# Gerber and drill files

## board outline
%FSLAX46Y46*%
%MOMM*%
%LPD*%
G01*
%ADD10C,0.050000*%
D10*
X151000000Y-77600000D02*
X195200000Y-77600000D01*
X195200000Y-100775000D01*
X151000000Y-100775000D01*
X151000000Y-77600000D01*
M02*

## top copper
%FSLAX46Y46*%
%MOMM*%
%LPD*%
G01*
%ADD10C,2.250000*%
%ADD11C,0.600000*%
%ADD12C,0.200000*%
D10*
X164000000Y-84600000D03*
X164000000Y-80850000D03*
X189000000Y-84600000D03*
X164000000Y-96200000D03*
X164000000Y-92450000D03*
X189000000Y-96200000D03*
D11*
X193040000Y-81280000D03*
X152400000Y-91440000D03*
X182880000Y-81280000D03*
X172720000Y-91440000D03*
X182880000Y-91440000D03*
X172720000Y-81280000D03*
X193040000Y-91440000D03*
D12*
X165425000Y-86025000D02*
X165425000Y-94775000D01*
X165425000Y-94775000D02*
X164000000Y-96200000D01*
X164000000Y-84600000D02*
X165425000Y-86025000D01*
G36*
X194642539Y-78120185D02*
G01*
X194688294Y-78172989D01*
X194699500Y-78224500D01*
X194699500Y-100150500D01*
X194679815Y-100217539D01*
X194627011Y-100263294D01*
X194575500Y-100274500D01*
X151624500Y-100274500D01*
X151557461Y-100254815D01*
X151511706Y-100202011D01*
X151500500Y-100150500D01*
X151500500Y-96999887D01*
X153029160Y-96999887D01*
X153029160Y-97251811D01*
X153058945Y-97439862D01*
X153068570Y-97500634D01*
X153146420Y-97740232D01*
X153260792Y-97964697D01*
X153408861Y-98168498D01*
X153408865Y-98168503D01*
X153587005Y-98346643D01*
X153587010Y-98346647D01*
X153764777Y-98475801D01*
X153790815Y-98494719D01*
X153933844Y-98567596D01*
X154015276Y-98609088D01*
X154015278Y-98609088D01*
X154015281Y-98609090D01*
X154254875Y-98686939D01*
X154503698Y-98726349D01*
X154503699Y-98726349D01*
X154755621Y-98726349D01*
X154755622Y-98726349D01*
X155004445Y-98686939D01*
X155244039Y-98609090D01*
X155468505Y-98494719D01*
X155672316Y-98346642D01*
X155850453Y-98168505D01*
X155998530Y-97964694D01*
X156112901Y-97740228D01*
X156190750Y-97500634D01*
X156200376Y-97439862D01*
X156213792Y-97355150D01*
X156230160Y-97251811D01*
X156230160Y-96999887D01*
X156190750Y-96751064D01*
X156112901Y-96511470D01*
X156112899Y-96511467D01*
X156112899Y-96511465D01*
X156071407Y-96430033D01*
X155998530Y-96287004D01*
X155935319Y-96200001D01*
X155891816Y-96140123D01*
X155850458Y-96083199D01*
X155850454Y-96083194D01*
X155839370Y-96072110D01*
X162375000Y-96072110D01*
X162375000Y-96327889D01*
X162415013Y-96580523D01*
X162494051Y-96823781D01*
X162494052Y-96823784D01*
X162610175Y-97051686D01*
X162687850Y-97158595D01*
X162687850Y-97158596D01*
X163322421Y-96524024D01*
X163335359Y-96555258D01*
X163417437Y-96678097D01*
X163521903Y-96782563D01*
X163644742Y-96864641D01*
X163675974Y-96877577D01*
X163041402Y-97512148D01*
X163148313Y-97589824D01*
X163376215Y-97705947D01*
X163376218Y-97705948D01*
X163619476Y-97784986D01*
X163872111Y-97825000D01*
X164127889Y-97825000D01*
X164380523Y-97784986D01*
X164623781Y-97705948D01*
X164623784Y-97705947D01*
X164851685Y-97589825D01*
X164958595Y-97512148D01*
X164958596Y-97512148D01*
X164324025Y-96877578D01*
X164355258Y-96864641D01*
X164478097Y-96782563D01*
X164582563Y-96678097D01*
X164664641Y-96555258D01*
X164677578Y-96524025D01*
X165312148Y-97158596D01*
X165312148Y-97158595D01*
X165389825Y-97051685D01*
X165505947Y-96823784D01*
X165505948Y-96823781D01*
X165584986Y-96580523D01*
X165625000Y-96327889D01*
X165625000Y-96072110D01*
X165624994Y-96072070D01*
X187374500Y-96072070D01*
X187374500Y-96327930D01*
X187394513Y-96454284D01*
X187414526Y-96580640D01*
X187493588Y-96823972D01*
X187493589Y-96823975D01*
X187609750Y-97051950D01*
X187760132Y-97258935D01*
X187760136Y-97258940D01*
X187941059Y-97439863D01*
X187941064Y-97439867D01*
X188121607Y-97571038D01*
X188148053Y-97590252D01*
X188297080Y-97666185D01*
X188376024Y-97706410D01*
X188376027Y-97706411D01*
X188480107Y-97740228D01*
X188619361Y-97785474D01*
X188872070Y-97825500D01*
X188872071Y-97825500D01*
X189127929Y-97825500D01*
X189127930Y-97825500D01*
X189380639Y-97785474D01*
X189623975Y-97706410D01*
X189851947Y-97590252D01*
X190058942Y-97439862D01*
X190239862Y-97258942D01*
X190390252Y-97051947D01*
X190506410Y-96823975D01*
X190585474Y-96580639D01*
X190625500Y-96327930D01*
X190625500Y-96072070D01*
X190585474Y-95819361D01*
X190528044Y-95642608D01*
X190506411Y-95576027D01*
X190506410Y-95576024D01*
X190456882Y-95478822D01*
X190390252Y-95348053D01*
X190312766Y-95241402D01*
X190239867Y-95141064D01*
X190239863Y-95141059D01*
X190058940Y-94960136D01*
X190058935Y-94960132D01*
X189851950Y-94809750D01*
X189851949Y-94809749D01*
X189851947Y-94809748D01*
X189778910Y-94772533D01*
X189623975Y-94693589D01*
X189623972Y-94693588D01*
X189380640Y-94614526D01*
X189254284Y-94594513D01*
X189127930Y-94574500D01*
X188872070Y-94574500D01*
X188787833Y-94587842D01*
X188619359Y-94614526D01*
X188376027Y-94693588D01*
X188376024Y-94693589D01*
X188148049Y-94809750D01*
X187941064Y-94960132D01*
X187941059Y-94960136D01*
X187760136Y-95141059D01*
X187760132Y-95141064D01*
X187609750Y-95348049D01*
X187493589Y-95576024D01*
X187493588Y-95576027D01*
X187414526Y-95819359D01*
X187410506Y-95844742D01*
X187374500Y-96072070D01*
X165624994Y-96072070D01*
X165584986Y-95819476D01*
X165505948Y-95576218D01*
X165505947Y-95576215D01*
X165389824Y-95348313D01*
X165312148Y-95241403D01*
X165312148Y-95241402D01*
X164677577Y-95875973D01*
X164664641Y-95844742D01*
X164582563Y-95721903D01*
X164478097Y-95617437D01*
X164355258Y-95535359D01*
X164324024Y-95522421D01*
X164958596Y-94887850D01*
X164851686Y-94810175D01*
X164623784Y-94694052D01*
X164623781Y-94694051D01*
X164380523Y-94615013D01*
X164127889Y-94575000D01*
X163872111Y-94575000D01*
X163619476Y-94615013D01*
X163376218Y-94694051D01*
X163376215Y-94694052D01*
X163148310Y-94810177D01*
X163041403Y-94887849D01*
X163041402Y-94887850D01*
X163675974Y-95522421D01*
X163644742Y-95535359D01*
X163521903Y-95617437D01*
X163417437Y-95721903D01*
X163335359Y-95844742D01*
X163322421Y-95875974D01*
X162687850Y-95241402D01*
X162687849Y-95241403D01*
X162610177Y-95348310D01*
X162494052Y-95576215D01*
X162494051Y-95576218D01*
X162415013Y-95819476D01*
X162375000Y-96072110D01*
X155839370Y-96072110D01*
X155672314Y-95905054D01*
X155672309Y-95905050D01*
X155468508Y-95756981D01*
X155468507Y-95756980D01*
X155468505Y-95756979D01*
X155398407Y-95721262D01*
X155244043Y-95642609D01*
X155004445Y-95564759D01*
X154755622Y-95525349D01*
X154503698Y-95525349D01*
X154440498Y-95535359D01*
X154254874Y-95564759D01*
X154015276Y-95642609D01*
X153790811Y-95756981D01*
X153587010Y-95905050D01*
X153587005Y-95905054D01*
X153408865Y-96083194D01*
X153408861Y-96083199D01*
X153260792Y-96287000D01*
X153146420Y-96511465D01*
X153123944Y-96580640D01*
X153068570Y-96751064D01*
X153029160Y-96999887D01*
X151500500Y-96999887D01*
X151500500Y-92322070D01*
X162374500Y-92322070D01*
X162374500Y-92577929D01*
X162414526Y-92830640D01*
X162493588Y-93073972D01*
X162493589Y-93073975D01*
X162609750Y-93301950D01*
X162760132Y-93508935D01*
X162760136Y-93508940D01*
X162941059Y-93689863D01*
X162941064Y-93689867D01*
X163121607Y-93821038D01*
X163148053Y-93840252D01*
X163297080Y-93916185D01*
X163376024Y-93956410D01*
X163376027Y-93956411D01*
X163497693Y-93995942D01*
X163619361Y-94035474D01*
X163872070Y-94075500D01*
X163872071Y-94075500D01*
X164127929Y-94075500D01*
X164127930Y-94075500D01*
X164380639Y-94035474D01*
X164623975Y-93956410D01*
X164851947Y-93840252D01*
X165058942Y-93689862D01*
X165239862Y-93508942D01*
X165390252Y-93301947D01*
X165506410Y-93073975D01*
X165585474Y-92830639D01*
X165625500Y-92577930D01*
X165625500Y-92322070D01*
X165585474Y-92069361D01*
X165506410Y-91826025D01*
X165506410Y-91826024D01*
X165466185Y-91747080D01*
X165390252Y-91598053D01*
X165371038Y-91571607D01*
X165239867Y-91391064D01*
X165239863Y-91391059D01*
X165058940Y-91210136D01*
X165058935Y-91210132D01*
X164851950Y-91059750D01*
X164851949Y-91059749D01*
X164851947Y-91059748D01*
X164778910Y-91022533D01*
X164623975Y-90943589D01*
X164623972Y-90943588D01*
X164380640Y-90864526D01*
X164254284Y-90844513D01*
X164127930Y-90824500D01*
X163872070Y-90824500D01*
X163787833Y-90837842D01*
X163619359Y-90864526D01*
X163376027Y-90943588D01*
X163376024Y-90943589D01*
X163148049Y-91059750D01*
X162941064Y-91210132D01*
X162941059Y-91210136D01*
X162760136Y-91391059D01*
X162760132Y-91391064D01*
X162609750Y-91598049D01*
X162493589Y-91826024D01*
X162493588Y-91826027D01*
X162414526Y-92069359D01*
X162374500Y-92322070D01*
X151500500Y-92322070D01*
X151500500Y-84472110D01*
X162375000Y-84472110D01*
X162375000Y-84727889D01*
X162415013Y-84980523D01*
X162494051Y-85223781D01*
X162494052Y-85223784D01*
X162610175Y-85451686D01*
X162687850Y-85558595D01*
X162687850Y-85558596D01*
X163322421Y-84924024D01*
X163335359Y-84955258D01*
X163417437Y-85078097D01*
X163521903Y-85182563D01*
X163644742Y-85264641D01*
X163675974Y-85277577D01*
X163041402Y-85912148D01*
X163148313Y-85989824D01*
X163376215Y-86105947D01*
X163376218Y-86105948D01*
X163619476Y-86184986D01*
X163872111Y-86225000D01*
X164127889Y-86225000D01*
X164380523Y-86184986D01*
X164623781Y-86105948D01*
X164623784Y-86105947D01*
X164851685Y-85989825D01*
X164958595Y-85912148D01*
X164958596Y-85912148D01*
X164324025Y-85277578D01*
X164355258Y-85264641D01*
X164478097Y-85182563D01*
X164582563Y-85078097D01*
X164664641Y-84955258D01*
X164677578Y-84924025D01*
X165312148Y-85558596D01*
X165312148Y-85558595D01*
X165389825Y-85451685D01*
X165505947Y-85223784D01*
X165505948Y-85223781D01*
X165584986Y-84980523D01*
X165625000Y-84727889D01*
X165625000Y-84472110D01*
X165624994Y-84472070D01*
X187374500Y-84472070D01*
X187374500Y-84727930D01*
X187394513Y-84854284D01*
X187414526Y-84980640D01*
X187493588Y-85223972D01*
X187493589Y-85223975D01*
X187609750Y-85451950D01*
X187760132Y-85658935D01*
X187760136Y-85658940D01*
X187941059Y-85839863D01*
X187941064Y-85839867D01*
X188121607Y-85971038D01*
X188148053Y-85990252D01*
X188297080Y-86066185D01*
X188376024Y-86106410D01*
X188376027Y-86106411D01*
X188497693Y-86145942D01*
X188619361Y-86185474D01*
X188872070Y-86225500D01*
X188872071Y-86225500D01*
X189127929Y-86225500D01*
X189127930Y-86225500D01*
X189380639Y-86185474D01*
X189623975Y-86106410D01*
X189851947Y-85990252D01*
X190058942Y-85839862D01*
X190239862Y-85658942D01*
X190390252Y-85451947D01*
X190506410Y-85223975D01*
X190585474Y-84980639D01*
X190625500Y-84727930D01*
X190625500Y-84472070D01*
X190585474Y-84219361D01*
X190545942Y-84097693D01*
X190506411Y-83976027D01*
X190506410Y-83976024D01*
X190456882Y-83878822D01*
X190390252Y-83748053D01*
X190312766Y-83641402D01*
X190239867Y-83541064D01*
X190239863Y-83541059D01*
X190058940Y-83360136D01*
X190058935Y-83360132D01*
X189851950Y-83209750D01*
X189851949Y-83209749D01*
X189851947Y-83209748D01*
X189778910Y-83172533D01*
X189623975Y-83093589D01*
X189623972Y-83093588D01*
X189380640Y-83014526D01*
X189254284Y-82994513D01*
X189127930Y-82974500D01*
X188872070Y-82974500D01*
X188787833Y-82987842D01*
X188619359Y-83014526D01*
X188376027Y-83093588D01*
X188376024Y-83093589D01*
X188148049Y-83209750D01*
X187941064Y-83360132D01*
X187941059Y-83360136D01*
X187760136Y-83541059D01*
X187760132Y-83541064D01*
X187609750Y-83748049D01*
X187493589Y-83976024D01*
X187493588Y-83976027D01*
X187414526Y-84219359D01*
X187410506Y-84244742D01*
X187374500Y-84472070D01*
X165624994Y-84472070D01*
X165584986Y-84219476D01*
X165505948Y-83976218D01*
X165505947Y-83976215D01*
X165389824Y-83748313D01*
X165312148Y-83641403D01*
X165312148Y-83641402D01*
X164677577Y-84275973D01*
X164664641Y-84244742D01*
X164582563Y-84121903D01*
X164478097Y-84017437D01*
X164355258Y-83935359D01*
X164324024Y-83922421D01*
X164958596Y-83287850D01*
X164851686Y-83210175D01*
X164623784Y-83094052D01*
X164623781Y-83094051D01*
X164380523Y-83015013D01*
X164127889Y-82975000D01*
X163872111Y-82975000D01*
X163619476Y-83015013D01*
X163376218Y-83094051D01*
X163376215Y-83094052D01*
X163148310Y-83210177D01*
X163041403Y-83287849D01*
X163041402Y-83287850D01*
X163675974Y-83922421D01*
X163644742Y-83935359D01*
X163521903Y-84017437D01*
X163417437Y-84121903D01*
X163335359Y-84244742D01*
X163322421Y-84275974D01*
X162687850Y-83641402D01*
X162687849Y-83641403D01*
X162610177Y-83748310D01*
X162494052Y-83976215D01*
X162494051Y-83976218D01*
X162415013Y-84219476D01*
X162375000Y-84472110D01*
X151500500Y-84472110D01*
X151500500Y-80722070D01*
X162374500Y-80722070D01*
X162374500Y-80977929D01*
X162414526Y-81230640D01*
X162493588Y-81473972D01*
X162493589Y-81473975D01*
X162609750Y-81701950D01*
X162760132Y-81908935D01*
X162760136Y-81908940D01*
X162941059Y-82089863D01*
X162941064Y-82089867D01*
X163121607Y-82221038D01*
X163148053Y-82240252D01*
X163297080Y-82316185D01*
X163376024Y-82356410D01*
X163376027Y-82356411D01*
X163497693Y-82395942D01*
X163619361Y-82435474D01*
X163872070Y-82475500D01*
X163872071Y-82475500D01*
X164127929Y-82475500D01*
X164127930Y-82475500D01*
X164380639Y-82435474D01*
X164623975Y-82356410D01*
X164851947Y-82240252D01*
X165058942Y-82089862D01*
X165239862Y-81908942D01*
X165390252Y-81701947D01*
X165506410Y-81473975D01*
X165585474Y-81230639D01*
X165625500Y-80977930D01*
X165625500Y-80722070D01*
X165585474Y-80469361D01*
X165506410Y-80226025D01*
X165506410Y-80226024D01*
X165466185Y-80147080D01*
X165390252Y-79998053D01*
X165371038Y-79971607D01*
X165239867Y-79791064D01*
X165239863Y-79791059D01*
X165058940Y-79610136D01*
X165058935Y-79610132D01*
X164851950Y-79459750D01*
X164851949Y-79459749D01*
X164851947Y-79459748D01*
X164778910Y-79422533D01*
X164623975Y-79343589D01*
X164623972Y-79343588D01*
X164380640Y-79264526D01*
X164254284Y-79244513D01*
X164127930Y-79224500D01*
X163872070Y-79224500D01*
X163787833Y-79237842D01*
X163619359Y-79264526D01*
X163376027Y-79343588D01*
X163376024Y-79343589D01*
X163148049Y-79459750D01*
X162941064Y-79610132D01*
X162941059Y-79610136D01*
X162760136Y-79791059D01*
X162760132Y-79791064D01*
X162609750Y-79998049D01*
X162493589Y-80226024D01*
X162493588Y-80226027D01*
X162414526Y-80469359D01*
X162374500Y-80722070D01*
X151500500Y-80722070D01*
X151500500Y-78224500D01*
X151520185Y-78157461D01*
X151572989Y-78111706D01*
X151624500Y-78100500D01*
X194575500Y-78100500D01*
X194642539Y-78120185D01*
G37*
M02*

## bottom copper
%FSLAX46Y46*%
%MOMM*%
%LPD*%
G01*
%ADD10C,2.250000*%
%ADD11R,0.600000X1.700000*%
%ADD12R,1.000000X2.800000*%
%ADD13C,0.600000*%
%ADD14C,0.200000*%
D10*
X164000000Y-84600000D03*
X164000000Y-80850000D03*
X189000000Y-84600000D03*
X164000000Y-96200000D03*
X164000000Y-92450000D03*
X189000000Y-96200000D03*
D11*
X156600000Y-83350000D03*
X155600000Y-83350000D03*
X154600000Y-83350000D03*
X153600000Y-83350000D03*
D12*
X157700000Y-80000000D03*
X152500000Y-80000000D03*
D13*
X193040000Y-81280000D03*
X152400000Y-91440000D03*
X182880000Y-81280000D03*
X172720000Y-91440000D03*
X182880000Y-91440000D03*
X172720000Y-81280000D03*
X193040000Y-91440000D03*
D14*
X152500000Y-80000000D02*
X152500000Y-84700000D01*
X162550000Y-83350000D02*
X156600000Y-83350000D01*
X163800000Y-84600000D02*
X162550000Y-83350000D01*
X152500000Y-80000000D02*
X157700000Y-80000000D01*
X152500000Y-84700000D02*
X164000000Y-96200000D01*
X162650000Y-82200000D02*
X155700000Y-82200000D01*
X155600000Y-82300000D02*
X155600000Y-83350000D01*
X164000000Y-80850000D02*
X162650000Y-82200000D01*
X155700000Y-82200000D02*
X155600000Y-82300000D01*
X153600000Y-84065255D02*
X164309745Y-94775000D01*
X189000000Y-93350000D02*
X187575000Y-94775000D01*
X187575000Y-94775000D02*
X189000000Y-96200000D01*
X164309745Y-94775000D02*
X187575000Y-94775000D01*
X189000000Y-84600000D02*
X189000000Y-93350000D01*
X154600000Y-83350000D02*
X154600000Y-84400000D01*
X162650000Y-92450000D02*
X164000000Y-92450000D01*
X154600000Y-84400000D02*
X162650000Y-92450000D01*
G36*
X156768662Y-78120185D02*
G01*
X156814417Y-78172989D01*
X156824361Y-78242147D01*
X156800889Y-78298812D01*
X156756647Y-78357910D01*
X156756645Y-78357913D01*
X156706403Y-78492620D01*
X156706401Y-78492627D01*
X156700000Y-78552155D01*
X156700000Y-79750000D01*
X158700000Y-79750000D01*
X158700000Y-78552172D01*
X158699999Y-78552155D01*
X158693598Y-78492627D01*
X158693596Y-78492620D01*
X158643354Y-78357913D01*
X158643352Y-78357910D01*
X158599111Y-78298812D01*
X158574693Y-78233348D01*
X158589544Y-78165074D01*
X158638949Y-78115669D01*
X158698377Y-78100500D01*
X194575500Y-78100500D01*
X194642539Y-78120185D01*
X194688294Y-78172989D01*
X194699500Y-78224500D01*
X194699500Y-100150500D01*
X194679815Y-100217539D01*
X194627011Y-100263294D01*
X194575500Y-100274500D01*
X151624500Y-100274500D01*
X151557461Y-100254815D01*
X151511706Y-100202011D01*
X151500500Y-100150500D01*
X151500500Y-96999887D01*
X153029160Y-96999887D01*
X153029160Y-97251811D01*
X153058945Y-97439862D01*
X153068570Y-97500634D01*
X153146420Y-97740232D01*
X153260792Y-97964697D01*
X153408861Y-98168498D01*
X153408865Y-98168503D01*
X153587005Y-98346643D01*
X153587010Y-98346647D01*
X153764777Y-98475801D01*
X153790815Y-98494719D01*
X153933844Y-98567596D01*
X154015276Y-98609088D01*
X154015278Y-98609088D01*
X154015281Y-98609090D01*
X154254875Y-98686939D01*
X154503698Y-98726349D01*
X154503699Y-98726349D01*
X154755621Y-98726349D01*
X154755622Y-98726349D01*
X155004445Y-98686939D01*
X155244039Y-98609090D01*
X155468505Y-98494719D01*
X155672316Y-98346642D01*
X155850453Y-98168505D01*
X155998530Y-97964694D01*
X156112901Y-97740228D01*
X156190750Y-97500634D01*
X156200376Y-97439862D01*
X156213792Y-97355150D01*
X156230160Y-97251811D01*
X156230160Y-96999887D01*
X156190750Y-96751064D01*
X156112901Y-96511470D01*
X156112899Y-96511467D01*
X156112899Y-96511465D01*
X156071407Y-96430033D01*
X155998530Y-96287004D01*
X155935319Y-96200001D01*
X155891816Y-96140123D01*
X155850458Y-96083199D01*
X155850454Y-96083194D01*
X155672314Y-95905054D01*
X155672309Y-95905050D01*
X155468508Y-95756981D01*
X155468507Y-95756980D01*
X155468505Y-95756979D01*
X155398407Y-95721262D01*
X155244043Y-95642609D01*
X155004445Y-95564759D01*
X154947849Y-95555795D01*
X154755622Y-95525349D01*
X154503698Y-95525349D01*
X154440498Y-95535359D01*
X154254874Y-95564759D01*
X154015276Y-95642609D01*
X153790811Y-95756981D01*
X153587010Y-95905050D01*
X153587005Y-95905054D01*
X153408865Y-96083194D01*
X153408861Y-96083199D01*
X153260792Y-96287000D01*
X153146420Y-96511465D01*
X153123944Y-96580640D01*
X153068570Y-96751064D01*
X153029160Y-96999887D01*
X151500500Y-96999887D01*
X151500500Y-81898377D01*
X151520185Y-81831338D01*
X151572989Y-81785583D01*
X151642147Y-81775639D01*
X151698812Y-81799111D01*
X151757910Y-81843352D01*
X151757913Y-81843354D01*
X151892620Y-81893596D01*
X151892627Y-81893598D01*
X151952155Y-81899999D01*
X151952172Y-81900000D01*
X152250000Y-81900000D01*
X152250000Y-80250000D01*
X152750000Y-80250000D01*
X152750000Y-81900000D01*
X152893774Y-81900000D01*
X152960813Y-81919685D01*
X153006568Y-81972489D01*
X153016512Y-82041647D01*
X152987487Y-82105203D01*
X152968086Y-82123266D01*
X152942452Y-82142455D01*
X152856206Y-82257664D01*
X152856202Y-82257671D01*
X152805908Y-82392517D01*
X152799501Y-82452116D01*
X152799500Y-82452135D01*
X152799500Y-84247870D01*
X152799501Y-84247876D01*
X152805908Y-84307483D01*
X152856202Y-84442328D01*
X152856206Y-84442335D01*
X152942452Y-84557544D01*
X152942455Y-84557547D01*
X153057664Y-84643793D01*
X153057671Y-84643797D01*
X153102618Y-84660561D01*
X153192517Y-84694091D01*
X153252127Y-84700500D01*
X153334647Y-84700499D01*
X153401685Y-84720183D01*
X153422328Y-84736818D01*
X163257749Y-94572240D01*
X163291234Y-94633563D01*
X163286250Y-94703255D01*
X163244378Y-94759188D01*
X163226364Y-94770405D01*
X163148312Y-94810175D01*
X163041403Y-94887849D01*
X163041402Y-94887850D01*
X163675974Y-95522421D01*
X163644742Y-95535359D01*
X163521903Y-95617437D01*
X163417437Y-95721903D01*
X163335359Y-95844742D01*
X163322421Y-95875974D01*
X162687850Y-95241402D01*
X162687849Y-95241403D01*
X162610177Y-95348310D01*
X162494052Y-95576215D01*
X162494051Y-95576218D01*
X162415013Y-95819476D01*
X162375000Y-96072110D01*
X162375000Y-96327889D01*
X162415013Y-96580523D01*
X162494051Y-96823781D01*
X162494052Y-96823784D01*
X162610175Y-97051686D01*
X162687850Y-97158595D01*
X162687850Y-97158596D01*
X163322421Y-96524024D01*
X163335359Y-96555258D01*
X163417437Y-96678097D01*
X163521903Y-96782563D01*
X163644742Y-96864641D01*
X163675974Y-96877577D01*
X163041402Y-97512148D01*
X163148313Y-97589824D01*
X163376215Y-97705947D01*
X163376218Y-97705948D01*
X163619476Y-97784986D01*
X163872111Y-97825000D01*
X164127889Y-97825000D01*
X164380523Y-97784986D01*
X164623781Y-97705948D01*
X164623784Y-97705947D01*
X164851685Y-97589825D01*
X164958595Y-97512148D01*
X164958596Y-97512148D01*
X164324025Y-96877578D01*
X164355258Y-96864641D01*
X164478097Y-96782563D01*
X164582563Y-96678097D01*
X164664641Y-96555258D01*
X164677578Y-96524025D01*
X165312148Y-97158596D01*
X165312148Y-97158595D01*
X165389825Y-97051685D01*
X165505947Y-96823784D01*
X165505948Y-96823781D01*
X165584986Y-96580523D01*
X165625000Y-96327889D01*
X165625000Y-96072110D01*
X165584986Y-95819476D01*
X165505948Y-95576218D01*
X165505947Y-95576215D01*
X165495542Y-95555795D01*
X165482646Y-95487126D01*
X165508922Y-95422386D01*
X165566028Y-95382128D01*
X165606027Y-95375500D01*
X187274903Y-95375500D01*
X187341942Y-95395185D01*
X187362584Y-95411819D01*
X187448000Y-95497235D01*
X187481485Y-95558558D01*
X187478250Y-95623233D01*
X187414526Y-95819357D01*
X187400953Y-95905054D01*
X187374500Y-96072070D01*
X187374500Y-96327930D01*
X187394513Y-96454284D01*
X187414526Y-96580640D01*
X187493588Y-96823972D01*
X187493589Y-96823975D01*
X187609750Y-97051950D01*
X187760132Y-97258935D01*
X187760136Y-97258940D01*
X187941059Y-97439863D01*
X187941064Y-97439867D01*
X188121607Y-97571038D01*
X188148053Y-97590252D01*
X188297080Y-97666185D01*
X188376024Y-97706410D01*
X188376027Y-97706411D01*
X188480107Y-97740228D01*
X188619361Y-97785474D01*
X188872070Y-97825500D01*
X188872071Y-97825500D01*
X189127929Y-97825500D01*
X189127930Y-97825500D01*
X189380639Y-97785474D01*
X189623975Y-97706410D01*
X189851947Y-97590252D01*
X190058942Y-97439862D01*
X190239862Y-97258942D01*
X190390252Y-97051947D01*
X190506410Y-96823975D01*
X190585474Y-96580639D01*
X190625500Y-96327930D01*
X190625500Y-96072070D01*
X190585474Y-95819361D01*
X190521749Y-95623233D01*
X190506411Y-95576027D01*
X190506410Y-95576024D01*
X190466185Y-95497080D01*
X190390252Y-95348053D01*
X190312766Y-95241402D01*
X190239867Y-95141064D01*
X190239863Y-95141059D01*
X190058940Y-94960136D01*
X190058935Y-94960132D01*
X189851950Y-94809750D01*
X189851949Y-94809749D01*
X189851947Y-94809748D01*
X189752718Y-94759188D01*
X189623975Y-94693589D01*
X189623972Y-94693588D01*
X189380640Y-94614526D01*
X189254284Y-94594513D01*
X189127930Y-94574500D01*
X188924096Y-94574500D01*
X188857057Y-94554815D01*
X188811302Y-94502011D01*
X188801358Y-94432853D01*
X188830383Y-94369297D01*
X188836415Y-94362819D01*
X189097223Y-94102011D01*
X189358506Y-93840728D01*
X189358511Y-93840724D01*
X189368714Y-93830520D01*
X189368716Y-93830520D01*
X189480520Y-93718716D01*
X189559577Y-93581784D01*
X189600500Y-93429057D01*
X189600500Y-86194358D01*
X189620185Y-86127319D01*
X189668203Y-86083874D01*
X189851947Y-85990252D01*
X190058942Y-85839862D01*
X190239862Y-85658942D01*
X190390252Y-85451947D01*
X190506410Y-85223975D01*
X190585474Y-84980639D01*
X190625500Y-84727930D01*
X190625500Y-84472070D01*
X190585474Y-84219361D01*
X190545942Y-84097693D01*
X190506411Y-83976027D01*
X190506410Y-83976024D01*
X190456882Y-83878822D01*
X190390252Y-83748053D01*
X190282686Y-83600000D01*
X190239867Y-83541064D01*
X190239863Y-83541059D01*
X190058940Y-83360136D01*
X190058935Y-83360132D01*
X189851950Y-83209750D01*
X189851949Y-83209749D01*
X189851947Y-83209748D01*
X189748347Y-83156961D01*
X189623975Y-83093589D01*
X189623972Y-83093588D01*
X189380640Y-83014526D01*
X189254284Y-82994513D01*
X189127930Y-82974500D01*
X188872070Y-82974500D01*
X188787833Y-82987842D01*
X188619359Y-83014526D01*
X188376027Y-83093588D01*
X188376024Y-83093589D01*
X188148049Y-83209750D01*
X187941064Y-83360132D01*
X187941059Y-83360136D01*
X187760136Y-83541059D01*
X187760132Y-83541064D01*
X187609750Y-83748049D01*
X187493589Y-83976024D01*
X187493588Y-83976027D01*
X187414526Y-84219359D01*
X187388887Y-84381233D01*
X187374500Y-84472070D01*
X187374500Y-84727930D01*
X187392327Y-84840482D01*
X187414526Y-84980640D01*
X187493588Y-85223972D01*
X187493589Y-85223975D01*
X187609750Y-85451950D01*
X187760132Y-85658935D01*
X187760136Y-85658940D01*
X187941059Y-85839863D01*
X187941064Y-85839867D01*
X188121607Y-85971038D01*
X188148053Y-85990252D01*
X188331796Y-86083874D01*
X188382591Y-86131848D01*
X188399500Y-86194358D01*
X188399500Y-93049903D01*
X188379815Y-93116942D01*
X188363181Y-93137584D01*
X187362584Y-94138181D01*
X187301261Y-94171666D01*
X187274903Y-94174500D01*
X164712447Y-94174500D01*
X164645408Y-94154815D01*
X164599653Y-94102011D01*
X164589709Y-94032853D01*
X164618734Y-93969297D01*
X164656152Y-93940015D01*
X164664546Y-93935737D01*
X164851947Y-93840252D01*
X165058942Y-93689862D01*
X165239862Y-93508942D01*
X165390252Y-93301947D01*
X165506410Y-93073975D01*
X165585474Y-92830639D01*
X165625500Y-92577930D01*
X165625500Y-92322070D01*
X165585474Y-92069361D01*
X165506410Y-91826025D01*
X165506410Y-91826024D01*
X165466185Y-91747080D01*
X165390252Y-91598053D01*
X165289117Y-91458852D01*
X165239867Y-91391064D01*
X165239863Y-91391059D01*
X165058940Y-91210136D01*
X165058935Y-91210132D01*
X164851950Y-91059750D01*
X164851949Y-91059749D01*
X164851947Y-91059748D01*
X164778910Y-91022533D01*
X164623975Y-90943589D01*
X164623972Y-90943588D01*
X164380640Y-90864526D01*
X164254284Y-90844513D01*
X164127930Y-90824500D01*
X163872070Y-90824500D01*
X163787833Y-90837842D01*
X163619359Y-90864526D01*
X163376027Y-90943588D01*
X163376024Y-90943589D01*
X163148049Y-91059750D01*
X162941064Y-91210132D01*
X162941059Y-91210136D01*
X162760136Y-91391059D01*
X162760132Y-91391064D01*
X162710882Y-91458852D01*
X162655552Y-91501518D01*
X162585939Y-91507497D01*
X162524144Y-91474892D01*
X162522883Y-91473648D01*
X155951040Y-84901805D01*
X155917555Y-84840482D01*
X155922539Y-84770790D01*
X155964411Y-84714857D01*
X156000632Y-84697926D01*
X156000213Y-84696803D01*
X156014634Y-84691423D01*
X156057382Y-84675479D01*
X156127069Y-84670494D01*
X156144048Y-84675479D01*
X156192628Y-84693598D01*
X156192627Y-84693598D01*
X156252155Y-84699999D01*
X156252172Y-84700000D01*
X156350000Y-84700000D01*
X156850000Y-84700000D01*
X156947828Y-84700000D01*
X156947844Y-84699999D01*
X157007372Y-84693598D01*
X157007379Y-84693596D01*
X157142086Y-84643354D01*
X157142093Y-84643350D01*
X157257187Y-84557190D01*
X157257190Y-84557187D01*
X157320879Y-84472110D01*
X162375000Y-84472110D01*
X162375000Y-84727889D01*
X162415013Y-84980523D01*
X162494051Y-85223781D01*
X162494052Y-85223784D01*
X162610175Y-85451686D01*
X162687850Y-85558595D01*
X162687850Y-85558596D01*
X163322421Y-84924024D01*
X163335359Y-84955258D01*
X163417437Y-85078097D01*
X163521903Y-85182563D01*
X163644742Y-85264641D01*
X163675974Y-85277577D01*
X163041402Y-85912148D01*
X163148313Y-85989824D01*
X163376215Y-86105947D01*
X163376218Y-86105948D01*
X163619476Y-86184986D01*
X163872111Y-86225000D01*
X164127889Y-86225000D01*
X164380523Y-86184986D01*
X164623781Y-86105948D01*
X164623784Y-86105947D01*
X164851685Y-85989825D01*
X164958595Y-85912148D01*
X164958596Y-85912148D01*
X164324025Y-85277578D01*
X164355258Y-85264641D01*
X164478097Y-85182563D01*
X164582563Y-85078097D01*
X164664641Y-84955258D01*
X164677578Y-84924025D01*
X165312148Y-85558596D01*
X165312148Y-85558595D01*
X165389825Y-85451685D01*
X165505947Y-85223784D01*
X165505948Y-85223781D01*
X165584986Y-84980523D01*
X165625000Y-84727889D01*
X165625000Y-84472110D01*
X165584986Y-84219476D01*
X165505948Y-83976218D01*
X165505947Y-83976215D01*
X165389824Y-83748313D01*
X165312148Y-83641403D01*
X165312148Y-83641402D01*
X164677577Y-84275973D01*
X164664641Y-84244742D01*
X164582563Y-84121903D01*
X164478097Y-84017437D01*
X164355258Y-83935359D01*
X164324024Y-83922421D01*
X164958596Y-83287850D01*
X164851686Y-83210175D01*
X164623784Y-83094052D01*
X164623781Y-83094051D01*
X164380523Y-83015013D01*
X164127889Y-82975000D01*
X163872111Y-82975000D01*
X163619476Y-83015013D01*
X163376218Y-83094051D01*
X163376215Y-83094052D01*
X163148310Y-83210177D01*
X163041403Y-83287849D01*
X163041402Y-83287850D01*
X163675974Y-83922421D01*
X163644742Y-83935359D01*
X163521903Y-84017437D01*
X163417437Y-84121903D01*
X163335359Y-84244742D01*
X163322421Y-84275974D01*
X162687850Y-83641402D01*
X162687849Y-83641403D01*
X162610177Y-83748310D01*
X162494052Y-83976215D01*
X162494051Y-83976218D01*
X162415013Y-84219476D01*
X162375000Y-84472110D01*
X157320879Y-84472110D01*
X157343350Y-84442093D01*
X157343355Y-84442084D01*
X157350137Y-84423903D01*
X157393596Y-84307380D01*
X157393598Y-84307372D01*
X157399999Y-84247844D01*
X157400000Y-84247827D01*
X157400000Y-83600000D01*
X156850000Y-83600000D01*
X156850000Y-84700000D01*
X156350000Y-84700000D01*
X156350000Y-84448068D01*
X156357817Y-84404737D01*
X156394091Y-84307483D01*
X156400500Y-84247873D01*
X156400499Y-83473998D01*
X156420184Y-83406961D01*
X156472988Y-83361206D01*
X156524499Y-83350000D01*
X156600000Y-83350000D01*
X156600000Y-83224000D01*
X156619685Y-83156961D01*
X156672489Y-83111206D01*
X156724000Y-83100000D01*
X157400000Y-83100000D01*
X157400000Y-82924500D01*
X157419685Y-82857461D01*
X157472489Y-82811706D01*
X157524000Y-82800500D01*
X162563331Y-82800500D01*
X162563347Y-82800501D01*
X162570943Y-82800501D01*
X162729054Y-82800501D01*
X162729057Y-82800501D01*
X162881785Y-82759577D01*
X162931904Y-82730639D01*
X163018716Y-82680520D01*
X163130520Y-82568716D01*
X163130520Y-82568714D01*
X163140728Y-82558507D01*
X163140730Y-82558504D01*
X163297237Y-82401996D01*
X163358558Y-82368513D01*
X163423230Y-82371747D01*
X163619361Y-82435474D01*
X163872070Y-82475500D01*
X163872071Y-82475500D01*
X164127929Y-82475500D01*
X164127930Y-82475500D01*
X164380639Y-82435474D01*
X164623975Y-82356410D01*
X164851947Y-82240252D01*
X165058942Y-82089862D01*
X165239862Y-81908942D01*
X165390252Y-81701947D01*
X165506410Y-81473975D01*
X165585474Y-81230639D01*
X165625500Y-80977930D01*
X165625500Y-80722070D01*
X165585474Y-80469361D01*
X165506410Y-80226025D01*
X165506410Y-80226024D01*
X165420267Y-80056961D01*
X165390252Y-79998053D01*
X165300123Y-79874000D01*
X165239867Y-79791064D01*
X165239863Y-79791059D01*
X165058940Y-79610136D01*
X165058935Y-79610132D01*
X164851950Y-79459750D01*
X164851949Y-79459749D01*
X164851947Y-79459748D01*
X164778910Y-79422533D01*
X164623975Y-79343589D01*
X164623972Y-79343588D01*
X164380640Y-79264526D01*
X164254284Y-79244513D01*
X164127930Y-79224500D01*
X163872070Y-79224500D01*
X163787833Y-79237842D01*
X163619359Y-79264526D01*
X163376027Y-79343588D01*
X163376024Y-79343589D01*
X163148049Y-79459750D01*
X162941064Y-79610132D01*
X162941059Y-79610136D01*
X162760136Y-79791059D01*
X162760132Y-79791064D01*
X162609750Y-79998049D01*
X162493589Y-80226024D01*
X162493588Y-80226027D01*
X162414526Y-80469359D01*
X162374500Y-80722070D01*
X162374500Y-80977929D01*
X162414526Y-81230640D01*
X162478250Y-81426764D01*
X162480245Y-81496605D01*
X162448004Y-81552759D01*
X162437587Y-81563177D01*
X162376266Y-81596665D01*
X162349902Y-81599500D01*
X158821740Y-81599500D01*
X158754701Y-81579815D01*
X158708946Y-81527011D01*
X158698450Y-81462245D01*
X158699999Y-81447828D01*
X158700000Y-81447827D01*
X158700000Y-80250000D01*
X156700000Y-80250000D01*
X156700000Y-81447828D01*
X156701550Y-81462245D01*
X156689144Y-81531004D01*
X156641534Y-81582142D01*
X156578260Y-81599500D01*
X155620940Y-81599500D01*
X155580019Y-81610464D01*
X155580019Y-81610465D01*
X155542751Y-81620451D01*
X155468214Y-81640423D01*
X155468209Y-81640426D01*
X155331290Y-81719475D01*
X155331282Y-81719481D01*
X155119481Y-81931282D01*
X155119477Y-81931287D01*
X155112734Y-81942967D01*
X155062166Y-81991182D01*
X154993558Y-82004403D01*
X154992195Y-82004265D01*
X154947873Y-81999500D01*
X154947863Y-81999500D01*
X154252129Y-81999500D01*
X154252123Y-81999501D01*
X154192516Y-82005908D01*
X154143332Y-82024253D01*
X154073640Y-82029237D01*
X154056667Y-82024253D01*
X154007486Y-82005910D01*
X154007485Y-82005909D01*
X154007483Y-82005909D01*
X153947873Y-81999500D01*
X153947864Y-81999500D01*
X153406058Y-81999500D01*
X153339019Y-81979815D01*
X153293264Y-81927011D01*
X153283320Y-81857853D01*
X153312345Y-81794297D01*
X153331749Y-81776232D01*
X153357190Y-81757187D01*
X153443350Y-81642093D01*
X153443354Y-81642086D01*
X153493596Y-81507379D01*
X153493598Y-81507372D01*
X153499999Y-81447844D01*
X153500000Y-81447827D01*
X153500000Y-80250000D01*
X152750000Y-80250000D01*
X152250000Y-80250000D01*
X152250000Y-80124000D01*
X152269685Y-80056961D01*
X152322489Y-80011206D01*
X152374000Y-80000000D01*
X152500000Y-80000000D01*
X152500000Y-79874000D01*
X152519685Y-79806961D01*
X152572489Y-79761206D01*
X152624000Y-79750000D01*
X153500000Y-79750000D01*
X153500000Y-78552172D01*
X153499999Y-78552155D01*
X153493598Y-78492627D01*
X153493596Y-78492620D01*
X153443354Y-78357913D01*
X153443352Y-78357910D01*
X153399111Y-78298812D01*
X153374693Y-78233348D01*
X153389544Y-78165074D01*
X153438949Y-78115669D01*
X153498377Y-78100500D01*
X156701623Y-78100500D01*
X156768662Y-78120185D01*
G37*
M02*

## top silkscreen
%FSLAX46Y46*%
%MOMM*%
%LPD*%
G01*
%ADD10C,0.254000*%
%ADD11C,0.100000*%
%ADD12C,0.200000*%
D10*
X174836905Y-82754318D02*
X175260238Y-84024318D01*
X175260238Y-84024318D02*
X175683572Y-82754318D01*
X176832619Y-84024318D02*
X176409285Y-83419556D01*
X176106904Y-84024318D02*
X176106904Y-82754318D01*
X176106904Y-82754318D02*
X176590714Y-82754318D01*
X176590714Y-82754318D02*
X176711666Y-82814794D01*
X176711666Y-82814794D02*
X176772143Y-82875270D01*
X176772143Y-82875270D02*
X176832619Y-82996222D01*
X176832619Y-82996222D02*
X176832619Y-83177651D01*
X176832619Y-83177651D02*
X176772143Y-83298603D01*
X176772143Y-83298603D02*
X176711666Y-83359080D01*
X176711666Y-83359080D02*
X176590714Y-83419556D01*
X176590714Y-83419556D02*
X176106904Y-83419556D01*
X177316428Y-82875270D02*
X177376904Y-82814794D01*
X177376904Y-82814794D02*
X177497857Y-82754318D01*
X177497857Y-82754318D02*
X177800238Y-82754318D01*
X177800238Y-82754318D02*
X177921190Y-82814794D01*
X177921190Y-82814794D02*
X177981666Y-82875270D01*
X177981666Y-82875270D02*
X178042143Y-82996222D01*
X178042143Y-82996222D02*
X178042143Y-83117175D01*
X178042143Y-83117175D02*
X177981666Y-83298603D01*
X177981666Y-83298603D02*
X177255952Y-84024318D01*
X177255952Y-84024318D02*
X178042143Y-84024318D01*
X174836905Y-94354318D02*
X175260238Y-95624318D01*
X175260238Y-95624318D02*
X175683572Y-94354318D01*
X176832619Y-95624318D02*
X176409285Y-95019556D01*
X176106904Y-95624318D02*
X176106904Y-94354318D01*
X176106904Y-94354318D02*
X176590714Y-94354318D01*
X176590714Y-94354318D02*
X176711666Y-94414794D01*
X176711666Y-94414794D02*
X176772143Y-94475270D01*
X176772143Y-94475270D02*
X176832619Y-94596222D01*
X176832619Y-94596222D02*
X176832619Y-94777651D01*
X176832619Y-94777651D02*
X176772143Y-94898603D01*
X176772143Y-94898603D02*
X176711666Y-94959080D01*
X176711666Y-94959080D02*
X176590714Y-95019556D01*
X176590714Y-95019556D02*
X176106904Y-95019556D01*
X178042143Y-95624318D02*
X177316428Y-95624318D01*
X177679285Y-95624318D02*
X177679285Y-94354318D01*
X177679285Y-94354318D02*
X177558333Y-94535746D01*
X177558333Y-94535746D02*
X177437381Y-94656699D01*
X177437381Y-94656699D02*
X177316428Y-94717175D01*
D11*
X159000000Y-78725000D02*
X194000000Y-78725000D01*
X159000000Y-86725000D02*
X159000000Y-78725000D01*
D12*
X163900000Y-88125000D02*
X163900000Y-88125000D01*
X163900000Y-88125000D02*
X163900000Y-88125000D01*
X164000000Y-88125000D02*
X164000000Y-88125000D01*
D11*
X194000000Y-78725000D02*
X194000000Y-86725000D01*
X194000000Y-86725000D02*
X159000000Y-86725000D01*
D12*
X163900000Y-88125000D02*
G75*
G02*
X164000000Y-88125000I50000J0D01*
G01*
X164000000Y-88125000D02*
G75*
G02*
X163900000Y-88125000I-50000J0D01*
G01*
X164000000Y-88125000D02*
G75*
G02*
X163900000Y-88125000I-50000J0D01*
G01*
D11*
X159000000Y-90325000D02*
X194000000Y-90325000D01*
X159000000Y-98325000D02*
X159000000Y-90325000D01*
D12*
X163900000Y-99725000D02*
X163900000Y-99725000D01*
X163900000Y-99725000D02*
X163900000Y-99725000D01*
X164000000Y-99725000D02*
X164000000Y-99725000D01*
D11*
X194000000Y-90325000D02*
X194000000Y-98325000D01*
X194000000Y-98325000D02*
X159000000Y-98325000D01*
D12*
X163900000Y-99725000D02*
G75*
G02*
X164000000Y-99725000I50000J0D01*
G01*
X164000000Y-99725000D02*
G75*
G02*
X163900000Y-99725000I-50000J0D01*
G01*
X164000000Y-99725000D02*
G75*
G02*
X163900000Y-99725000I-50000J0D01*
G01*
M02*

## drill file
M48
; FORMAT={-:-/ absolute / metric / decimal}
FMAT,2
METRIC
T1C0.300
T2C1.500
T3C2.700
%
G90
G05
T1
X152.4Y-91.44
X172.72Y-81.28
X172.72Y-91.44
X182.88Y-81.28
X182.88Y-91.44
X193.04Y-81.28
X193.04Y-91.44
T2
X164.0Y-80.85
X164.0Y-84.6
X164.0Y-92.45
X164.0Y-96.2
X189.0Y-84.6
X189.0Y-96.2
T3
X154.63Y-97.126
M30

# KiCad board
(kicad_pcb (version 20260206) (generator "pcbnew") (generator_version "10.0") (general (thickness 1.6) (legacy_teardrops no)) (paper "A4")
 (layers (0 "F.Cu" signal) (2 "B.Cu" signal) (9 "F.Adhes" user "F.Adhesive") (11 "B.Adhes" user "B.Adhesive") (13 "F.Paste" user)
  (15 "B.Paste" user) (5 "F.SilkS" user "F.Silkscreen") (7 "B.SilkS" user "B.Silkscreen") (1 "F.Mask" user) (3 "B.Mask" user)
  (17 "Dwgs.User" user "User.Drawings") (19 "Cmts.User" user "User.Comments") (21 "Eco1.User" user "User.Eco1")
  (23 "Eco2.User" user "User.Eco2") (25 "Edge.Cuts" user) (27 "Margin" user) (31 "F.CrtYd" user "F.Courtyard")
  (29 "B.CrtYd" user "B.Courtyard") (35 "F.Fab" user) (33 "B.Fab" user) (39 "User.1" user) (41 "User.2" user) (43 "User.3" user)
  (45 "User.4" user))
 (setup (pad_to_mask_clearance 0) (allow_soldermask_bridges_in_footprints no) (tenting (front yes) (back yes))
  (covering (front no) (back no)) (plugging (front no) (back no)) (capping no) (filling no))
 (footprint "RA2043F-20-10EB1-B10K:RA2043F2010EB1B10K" (layer "F.Cu") (at 164 84.6)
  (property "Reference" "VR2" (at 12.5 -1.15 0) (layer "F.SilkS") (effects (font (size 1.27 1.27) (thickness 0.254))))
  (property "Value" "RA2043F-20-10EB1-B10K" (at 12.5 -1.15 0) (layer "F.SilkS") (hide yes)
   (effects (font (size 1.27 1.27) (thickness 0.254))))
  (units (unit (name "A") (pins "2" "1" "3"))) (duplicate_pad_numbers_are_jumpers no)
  (fp_line (start -5 -5.875) (end 30 -5.875) (stroke (width 0.1) (type solid)) (layer "F.SilkS"))
  (fp_line (start -5 2.125) (end -5 -5.875) (stroke (width 0.1) (type solid)) (layer "F.SilkS"))
  (fp_line (start -0.1 3.525) (end -0.1 3.525) (stroke (width 0.2) (type solid)) (layer "F.SilkS"))
  (fp_line (start -0.1 3.525) (end -0.1 3.525) (stroke (width 0.2) (type solid)) (layer "F.SilkS"))
  (fp_line (start 0 3.525) (end 0 3.525) (stroke (width 0.2) (type solid)) (layer "F.SilkS"))
  (fp_line (start 30 -5.875) (end 30 2.125) (stroke (width 0.1) (type solid)) (layer "F.SilkS"))
  (fp_line (start 30 2.125) (end -5 2.125) (stroke (width 0.1) (type solid)) (layer "F.SilkS"))
  (fp_arc (start -0.1 3.525) (mid -0.05 3.475) (end 0 3.525) (stroke (width 0.2) (type solid)) (layer "F.SilkS"))
  (fp_arc (start 0 3.525) (mid -0.05 3.575) (end -0.1 3.525) (stroke (width 0.2) (type solid)) (layer "F.SilkS"))
  (fp_arc (start 0 3.525) (mid -0.05 3.575) (end -0.1 3.525) (stroke (width 0.2) (type solid)) (layer "F.SilkS"))
  (pad "1" thru_hole circle (at 0 0) (size 2.25 2.25) (drill 1.5) (layers "*.Cu" "*.Mask") (remove_unused_layers no) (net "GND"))
  (pad "2" thru_hole circle (at 0 -3.75) (size 2.25 2.25) (drill 1.5) (layers "*.Cu" "*.Mask") (remove_unused_layers no) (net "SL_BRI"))
  (pad "3" thru_hole circle (at 25 0) (size 2.25 2.25) (drill 1.5) (layers "*.Cu" "*.Mask") (remove_unused_layers no) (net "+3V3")))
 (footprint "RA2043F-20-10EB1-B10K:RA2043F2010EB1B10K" (layer "F.Cu") (at 164 96.2)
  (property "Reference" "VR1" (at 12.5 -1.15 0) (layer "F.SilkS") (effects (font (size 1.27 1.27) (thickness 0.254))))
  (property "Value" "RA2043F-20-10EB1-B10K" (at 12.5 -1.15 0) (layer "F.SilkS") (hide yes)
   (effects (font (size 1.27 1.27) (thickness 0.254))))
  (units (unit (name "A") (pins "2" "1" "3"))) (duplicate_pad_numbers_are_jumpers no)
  (fp_line (start -5 -5.875) (end 30 -5.875) (stroke (width 0.1) (type solid)) (layer "F.SilkS"))
  (fp_line (start -5 2.125) (end -5 -5.875) (stroke (width 0.1) (type solid)) (layer "F.SilkS"))
  (fp_line (start -0.1 3.525) (end -0.1 3.525) (stroke (width 0.2) (type solid)) (layer "F.SilkS"))
  (fp_line (start -0.1 3.525) (end -0.1 3.525) (stroke (width 0.2) (type solid)) (layer "F.SilkS"))
  (fp_line (start 0 3.525) (end 0 3.525) (stroke (width 0.2) (type solid)) (layer "F.SilkS"))
  (fp_line (start 30 -5.875) (end 30 2.125) (stroke (width 0.1) (type solid)) (layer "F.SilkS"))
  (fp_line (start 30 2.125) (end -5 2.125) (stroke (width 0.1) (type solid)) (layer "F.SilkS"))
  (fp_arc (start -0.1 3.525) (mid -0.05 3.475) (end 0 3.525) (stroke (width 0.2) (type solid)) (layer "F.SilkS"))
  (fp_arc (start 0 3.525) (mid -0.05 3.575) (end -0.1 3.525) (stroke (width 0.2) (type solid)) (layer "F.SilkS"))
  (fp_arc (start 0 3.525) (mid -0.05 3.575) (end -0.1 3.525) (stroke (width 0.2) (type solid)) (layer "F.SilkS"))
  (pad "1" thru_hole circle (at 0 0) (size 2.25 2.25) (drill 1.5) (layers "*.Cu" "*.Mask") (remove_unused_layers no) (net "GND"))
  (pad "2" thru_hole circle (at 0 -3.75) (size 2.25 2.25) (drill 1.5) (layers "*.Cu" "*.Mask") (remove_unused_layers no) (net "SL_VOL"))
  (pad "3" thru_hole circle (at 25 0) (size 2.25 2.25) (drill 1.5) (layers "*.Cu" "*.Mask") (remove_unused_layers no) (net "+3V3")))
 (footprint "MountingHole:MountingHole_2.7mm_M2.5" (layer "B.Cu") (at 154.62966 97.125849 -90)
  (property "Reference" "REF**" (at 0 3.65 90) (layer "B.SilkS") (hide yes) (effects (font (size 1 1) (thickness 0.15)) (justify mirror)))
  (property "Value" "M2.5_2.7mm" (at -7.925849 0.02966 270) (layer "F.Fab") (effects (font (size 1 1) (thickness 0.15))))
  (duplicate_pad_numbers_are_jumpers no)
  (pad "" np_thru_hole circle (at 0 0 270) (size 2.7 2.7) (drill 2.7) (layers "*.Cu" "*.Mask")))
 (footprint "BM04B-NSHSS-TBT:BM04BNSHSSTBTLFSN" (layer "B.Cu") (at 155.1 81.125)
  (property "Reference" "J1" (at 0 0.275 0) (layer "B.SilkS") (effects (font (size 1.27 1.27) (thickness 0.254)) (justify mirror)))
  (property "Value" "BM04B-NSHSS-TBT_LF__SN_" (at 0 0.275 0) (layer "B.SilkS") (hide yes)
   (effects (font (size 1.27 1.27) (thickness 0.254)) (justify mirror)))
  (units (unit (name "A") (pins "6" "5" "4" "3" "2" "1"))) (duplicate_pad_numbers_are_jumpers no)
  (pad "1" smd rect (at 1.5 2.225) (size 0.6 1.7) (layers "B.Cu" "B.Mask" "B.Paste") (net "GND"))
  (pad "2" smd rect (at 0.5 2.225) (size 0.6 1.7) (layers "B.Cu" "B.Mask" "B.Paste") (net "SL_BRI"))
  (pad "3" smd rect (at -0.5 2.225) (size 0.6 1.7) (layers "B.Cu" "B.Mask" "B.Paste") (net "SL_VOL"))
  (pad "4" smd rect (at -1.5 2.225) (size 0.6 1.7) (layers "B.Cu" "B.Mask" "B.Paste") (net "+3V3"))
  (pad "5" smd rect (at 2.6 -1.125) (size 1 2.8) (layers "B.Cu" "B.Mask" "B.Paste") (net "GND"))
  (pad "6" smd rect (at -2.6 -1.125) (size 1 2.8) (layers "B.Cu" "B.Mask" "B.Paste") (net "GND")))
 (gr_rect (start 151 77.6) (end 195.2 100.775) (stroke (width 0.05) (type solid)) (fill no) (layer "Edge.Cuts"))
 (segment (start 165.425 86.025) (end 165.425 94.775) (width 0.2) (layer "F.Cu") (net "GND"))
 (segment (start 165.425 94.775) (end 164 96.2) (width 0.2) (layer "F.Cu") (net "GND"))
 (segment (start 164 84.6) (end 165.425 86.025) (width 0.2) (layer "F.Cu") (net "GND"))
 (via (at 193.04 81.28) (size 0.6) (drill 0.3) (layers "F.Cu" "B.Cu") (free yes) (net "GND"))
 (via (at 152.4 91.44) (size 0.6) (drill 0.3) (layers "F.Cu" "B.Cu") (free yes) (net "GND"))
 (via (at 182.88 81.28) (size 0.6) (drill 0.3) (layers "F.Cu" "B.Cu") (free yes) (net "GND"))
 (via (at 172.72 91.44) (size 0.6) (drill 0.3) (layers "F.Cu" "B.Cu") (free yes) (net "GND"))
 (via (at 182.88 91.44) (size 0.6) (drill 0.3) (layers "F.Cu" "B.Cu") (free yes) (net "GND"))
 (via (at 172.72 81.28) (size 0.6) (drill 0.3) (layers "F.Cu" "B.Cu") (free yes) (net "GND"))
 (via (at 193.04 91.44) (size 0.6) (drill 0.3) (layers "F.Cu" "B.Cu") (free yes) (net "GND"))
 (segment (start 152.5 80) (end 152.5 84.7) (width 0.2) (layer "B.Cu") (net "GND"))
 (segment (start 162.55 83.35) (end 156.6 83.35) (width 0.2) (layer "B.Cu") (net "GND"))
 (segment (start 163.8 84.6) (end 162.55 83.35) (width 0.2) (layer "B.Cu") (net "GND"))
 (segment (start 152.5 80) (end 157.7 80) (width 0.2) (layer "B.Cu") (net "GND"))
 (segment (start 152.5 84.7) (end 164 96.2) (width 0.2) (layer "B.Cu") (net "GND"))
 (segment (start 162.65 82.2) (end 155.7 82.2) (width 0.2) (layer "B.Cu") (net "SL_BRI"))
 (segment (start 155.6 82.3) (end 155.6 83.35) (width 0.2) (layer "B.Cu") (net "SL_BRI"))
 (segment (start 164 80.85) (end 162.65 82.2) (width 0.2) (layer "B.Cu") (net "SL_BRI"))
 (segment (start 155.7 82.2) (end 155.6 82.3) (width 0.2) (layer "B.Cu") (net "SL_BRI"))
 (segment (start 153.6 84.065255) (end 164.309745 94.775) (width 0.2) (layer "B.Cu") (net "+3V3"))
 (segment (start 189 93.35) (end 187.575 94.775) (width 0.2) (layer "B.Cu") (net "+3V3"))
 (segment (start 187.575 94.775) (end 189 96.2) (width 0.2) (layer "B.Cu") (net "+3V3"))
 (segment (start 164.309745 94.775) (end 187.575 94.775) (width 0.2) (layer "B.Cu") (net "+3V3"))
 (segment (start 189 84.6) (end 189 93.35) (width 0.2) (layer "B.Cu") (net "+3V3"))
 (segment (start 154.6 83.35) (end 154.6 84.4) (width 0.2) (layer "B.Cu") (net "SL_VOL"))
 (segment (start 162.65 92.45) (end 164 92.45) (width 0.2) (layer "B.Cu") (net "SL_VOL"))
 (segment (start 154.6 84.4) (end 162.65 92.45) (width 0.2) (layer "B.Cu") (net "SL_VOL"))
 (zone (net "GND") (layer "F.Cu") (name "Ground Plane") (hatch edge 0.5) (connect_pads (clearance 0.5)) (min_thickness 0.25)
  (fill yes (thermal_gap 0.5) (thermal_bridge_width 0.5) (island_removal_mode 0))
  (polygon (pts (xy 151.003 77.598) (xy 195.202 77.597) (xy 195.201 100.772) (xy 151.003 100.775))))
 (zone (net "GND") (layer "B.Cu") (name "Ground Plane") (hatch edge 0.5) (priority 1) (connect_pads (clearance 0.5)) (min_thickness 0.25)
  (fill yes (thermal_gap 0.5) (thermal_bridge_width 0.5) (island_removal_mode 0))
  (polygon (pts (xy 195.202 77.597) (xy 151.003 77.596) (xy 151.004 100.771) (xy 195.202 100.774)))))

